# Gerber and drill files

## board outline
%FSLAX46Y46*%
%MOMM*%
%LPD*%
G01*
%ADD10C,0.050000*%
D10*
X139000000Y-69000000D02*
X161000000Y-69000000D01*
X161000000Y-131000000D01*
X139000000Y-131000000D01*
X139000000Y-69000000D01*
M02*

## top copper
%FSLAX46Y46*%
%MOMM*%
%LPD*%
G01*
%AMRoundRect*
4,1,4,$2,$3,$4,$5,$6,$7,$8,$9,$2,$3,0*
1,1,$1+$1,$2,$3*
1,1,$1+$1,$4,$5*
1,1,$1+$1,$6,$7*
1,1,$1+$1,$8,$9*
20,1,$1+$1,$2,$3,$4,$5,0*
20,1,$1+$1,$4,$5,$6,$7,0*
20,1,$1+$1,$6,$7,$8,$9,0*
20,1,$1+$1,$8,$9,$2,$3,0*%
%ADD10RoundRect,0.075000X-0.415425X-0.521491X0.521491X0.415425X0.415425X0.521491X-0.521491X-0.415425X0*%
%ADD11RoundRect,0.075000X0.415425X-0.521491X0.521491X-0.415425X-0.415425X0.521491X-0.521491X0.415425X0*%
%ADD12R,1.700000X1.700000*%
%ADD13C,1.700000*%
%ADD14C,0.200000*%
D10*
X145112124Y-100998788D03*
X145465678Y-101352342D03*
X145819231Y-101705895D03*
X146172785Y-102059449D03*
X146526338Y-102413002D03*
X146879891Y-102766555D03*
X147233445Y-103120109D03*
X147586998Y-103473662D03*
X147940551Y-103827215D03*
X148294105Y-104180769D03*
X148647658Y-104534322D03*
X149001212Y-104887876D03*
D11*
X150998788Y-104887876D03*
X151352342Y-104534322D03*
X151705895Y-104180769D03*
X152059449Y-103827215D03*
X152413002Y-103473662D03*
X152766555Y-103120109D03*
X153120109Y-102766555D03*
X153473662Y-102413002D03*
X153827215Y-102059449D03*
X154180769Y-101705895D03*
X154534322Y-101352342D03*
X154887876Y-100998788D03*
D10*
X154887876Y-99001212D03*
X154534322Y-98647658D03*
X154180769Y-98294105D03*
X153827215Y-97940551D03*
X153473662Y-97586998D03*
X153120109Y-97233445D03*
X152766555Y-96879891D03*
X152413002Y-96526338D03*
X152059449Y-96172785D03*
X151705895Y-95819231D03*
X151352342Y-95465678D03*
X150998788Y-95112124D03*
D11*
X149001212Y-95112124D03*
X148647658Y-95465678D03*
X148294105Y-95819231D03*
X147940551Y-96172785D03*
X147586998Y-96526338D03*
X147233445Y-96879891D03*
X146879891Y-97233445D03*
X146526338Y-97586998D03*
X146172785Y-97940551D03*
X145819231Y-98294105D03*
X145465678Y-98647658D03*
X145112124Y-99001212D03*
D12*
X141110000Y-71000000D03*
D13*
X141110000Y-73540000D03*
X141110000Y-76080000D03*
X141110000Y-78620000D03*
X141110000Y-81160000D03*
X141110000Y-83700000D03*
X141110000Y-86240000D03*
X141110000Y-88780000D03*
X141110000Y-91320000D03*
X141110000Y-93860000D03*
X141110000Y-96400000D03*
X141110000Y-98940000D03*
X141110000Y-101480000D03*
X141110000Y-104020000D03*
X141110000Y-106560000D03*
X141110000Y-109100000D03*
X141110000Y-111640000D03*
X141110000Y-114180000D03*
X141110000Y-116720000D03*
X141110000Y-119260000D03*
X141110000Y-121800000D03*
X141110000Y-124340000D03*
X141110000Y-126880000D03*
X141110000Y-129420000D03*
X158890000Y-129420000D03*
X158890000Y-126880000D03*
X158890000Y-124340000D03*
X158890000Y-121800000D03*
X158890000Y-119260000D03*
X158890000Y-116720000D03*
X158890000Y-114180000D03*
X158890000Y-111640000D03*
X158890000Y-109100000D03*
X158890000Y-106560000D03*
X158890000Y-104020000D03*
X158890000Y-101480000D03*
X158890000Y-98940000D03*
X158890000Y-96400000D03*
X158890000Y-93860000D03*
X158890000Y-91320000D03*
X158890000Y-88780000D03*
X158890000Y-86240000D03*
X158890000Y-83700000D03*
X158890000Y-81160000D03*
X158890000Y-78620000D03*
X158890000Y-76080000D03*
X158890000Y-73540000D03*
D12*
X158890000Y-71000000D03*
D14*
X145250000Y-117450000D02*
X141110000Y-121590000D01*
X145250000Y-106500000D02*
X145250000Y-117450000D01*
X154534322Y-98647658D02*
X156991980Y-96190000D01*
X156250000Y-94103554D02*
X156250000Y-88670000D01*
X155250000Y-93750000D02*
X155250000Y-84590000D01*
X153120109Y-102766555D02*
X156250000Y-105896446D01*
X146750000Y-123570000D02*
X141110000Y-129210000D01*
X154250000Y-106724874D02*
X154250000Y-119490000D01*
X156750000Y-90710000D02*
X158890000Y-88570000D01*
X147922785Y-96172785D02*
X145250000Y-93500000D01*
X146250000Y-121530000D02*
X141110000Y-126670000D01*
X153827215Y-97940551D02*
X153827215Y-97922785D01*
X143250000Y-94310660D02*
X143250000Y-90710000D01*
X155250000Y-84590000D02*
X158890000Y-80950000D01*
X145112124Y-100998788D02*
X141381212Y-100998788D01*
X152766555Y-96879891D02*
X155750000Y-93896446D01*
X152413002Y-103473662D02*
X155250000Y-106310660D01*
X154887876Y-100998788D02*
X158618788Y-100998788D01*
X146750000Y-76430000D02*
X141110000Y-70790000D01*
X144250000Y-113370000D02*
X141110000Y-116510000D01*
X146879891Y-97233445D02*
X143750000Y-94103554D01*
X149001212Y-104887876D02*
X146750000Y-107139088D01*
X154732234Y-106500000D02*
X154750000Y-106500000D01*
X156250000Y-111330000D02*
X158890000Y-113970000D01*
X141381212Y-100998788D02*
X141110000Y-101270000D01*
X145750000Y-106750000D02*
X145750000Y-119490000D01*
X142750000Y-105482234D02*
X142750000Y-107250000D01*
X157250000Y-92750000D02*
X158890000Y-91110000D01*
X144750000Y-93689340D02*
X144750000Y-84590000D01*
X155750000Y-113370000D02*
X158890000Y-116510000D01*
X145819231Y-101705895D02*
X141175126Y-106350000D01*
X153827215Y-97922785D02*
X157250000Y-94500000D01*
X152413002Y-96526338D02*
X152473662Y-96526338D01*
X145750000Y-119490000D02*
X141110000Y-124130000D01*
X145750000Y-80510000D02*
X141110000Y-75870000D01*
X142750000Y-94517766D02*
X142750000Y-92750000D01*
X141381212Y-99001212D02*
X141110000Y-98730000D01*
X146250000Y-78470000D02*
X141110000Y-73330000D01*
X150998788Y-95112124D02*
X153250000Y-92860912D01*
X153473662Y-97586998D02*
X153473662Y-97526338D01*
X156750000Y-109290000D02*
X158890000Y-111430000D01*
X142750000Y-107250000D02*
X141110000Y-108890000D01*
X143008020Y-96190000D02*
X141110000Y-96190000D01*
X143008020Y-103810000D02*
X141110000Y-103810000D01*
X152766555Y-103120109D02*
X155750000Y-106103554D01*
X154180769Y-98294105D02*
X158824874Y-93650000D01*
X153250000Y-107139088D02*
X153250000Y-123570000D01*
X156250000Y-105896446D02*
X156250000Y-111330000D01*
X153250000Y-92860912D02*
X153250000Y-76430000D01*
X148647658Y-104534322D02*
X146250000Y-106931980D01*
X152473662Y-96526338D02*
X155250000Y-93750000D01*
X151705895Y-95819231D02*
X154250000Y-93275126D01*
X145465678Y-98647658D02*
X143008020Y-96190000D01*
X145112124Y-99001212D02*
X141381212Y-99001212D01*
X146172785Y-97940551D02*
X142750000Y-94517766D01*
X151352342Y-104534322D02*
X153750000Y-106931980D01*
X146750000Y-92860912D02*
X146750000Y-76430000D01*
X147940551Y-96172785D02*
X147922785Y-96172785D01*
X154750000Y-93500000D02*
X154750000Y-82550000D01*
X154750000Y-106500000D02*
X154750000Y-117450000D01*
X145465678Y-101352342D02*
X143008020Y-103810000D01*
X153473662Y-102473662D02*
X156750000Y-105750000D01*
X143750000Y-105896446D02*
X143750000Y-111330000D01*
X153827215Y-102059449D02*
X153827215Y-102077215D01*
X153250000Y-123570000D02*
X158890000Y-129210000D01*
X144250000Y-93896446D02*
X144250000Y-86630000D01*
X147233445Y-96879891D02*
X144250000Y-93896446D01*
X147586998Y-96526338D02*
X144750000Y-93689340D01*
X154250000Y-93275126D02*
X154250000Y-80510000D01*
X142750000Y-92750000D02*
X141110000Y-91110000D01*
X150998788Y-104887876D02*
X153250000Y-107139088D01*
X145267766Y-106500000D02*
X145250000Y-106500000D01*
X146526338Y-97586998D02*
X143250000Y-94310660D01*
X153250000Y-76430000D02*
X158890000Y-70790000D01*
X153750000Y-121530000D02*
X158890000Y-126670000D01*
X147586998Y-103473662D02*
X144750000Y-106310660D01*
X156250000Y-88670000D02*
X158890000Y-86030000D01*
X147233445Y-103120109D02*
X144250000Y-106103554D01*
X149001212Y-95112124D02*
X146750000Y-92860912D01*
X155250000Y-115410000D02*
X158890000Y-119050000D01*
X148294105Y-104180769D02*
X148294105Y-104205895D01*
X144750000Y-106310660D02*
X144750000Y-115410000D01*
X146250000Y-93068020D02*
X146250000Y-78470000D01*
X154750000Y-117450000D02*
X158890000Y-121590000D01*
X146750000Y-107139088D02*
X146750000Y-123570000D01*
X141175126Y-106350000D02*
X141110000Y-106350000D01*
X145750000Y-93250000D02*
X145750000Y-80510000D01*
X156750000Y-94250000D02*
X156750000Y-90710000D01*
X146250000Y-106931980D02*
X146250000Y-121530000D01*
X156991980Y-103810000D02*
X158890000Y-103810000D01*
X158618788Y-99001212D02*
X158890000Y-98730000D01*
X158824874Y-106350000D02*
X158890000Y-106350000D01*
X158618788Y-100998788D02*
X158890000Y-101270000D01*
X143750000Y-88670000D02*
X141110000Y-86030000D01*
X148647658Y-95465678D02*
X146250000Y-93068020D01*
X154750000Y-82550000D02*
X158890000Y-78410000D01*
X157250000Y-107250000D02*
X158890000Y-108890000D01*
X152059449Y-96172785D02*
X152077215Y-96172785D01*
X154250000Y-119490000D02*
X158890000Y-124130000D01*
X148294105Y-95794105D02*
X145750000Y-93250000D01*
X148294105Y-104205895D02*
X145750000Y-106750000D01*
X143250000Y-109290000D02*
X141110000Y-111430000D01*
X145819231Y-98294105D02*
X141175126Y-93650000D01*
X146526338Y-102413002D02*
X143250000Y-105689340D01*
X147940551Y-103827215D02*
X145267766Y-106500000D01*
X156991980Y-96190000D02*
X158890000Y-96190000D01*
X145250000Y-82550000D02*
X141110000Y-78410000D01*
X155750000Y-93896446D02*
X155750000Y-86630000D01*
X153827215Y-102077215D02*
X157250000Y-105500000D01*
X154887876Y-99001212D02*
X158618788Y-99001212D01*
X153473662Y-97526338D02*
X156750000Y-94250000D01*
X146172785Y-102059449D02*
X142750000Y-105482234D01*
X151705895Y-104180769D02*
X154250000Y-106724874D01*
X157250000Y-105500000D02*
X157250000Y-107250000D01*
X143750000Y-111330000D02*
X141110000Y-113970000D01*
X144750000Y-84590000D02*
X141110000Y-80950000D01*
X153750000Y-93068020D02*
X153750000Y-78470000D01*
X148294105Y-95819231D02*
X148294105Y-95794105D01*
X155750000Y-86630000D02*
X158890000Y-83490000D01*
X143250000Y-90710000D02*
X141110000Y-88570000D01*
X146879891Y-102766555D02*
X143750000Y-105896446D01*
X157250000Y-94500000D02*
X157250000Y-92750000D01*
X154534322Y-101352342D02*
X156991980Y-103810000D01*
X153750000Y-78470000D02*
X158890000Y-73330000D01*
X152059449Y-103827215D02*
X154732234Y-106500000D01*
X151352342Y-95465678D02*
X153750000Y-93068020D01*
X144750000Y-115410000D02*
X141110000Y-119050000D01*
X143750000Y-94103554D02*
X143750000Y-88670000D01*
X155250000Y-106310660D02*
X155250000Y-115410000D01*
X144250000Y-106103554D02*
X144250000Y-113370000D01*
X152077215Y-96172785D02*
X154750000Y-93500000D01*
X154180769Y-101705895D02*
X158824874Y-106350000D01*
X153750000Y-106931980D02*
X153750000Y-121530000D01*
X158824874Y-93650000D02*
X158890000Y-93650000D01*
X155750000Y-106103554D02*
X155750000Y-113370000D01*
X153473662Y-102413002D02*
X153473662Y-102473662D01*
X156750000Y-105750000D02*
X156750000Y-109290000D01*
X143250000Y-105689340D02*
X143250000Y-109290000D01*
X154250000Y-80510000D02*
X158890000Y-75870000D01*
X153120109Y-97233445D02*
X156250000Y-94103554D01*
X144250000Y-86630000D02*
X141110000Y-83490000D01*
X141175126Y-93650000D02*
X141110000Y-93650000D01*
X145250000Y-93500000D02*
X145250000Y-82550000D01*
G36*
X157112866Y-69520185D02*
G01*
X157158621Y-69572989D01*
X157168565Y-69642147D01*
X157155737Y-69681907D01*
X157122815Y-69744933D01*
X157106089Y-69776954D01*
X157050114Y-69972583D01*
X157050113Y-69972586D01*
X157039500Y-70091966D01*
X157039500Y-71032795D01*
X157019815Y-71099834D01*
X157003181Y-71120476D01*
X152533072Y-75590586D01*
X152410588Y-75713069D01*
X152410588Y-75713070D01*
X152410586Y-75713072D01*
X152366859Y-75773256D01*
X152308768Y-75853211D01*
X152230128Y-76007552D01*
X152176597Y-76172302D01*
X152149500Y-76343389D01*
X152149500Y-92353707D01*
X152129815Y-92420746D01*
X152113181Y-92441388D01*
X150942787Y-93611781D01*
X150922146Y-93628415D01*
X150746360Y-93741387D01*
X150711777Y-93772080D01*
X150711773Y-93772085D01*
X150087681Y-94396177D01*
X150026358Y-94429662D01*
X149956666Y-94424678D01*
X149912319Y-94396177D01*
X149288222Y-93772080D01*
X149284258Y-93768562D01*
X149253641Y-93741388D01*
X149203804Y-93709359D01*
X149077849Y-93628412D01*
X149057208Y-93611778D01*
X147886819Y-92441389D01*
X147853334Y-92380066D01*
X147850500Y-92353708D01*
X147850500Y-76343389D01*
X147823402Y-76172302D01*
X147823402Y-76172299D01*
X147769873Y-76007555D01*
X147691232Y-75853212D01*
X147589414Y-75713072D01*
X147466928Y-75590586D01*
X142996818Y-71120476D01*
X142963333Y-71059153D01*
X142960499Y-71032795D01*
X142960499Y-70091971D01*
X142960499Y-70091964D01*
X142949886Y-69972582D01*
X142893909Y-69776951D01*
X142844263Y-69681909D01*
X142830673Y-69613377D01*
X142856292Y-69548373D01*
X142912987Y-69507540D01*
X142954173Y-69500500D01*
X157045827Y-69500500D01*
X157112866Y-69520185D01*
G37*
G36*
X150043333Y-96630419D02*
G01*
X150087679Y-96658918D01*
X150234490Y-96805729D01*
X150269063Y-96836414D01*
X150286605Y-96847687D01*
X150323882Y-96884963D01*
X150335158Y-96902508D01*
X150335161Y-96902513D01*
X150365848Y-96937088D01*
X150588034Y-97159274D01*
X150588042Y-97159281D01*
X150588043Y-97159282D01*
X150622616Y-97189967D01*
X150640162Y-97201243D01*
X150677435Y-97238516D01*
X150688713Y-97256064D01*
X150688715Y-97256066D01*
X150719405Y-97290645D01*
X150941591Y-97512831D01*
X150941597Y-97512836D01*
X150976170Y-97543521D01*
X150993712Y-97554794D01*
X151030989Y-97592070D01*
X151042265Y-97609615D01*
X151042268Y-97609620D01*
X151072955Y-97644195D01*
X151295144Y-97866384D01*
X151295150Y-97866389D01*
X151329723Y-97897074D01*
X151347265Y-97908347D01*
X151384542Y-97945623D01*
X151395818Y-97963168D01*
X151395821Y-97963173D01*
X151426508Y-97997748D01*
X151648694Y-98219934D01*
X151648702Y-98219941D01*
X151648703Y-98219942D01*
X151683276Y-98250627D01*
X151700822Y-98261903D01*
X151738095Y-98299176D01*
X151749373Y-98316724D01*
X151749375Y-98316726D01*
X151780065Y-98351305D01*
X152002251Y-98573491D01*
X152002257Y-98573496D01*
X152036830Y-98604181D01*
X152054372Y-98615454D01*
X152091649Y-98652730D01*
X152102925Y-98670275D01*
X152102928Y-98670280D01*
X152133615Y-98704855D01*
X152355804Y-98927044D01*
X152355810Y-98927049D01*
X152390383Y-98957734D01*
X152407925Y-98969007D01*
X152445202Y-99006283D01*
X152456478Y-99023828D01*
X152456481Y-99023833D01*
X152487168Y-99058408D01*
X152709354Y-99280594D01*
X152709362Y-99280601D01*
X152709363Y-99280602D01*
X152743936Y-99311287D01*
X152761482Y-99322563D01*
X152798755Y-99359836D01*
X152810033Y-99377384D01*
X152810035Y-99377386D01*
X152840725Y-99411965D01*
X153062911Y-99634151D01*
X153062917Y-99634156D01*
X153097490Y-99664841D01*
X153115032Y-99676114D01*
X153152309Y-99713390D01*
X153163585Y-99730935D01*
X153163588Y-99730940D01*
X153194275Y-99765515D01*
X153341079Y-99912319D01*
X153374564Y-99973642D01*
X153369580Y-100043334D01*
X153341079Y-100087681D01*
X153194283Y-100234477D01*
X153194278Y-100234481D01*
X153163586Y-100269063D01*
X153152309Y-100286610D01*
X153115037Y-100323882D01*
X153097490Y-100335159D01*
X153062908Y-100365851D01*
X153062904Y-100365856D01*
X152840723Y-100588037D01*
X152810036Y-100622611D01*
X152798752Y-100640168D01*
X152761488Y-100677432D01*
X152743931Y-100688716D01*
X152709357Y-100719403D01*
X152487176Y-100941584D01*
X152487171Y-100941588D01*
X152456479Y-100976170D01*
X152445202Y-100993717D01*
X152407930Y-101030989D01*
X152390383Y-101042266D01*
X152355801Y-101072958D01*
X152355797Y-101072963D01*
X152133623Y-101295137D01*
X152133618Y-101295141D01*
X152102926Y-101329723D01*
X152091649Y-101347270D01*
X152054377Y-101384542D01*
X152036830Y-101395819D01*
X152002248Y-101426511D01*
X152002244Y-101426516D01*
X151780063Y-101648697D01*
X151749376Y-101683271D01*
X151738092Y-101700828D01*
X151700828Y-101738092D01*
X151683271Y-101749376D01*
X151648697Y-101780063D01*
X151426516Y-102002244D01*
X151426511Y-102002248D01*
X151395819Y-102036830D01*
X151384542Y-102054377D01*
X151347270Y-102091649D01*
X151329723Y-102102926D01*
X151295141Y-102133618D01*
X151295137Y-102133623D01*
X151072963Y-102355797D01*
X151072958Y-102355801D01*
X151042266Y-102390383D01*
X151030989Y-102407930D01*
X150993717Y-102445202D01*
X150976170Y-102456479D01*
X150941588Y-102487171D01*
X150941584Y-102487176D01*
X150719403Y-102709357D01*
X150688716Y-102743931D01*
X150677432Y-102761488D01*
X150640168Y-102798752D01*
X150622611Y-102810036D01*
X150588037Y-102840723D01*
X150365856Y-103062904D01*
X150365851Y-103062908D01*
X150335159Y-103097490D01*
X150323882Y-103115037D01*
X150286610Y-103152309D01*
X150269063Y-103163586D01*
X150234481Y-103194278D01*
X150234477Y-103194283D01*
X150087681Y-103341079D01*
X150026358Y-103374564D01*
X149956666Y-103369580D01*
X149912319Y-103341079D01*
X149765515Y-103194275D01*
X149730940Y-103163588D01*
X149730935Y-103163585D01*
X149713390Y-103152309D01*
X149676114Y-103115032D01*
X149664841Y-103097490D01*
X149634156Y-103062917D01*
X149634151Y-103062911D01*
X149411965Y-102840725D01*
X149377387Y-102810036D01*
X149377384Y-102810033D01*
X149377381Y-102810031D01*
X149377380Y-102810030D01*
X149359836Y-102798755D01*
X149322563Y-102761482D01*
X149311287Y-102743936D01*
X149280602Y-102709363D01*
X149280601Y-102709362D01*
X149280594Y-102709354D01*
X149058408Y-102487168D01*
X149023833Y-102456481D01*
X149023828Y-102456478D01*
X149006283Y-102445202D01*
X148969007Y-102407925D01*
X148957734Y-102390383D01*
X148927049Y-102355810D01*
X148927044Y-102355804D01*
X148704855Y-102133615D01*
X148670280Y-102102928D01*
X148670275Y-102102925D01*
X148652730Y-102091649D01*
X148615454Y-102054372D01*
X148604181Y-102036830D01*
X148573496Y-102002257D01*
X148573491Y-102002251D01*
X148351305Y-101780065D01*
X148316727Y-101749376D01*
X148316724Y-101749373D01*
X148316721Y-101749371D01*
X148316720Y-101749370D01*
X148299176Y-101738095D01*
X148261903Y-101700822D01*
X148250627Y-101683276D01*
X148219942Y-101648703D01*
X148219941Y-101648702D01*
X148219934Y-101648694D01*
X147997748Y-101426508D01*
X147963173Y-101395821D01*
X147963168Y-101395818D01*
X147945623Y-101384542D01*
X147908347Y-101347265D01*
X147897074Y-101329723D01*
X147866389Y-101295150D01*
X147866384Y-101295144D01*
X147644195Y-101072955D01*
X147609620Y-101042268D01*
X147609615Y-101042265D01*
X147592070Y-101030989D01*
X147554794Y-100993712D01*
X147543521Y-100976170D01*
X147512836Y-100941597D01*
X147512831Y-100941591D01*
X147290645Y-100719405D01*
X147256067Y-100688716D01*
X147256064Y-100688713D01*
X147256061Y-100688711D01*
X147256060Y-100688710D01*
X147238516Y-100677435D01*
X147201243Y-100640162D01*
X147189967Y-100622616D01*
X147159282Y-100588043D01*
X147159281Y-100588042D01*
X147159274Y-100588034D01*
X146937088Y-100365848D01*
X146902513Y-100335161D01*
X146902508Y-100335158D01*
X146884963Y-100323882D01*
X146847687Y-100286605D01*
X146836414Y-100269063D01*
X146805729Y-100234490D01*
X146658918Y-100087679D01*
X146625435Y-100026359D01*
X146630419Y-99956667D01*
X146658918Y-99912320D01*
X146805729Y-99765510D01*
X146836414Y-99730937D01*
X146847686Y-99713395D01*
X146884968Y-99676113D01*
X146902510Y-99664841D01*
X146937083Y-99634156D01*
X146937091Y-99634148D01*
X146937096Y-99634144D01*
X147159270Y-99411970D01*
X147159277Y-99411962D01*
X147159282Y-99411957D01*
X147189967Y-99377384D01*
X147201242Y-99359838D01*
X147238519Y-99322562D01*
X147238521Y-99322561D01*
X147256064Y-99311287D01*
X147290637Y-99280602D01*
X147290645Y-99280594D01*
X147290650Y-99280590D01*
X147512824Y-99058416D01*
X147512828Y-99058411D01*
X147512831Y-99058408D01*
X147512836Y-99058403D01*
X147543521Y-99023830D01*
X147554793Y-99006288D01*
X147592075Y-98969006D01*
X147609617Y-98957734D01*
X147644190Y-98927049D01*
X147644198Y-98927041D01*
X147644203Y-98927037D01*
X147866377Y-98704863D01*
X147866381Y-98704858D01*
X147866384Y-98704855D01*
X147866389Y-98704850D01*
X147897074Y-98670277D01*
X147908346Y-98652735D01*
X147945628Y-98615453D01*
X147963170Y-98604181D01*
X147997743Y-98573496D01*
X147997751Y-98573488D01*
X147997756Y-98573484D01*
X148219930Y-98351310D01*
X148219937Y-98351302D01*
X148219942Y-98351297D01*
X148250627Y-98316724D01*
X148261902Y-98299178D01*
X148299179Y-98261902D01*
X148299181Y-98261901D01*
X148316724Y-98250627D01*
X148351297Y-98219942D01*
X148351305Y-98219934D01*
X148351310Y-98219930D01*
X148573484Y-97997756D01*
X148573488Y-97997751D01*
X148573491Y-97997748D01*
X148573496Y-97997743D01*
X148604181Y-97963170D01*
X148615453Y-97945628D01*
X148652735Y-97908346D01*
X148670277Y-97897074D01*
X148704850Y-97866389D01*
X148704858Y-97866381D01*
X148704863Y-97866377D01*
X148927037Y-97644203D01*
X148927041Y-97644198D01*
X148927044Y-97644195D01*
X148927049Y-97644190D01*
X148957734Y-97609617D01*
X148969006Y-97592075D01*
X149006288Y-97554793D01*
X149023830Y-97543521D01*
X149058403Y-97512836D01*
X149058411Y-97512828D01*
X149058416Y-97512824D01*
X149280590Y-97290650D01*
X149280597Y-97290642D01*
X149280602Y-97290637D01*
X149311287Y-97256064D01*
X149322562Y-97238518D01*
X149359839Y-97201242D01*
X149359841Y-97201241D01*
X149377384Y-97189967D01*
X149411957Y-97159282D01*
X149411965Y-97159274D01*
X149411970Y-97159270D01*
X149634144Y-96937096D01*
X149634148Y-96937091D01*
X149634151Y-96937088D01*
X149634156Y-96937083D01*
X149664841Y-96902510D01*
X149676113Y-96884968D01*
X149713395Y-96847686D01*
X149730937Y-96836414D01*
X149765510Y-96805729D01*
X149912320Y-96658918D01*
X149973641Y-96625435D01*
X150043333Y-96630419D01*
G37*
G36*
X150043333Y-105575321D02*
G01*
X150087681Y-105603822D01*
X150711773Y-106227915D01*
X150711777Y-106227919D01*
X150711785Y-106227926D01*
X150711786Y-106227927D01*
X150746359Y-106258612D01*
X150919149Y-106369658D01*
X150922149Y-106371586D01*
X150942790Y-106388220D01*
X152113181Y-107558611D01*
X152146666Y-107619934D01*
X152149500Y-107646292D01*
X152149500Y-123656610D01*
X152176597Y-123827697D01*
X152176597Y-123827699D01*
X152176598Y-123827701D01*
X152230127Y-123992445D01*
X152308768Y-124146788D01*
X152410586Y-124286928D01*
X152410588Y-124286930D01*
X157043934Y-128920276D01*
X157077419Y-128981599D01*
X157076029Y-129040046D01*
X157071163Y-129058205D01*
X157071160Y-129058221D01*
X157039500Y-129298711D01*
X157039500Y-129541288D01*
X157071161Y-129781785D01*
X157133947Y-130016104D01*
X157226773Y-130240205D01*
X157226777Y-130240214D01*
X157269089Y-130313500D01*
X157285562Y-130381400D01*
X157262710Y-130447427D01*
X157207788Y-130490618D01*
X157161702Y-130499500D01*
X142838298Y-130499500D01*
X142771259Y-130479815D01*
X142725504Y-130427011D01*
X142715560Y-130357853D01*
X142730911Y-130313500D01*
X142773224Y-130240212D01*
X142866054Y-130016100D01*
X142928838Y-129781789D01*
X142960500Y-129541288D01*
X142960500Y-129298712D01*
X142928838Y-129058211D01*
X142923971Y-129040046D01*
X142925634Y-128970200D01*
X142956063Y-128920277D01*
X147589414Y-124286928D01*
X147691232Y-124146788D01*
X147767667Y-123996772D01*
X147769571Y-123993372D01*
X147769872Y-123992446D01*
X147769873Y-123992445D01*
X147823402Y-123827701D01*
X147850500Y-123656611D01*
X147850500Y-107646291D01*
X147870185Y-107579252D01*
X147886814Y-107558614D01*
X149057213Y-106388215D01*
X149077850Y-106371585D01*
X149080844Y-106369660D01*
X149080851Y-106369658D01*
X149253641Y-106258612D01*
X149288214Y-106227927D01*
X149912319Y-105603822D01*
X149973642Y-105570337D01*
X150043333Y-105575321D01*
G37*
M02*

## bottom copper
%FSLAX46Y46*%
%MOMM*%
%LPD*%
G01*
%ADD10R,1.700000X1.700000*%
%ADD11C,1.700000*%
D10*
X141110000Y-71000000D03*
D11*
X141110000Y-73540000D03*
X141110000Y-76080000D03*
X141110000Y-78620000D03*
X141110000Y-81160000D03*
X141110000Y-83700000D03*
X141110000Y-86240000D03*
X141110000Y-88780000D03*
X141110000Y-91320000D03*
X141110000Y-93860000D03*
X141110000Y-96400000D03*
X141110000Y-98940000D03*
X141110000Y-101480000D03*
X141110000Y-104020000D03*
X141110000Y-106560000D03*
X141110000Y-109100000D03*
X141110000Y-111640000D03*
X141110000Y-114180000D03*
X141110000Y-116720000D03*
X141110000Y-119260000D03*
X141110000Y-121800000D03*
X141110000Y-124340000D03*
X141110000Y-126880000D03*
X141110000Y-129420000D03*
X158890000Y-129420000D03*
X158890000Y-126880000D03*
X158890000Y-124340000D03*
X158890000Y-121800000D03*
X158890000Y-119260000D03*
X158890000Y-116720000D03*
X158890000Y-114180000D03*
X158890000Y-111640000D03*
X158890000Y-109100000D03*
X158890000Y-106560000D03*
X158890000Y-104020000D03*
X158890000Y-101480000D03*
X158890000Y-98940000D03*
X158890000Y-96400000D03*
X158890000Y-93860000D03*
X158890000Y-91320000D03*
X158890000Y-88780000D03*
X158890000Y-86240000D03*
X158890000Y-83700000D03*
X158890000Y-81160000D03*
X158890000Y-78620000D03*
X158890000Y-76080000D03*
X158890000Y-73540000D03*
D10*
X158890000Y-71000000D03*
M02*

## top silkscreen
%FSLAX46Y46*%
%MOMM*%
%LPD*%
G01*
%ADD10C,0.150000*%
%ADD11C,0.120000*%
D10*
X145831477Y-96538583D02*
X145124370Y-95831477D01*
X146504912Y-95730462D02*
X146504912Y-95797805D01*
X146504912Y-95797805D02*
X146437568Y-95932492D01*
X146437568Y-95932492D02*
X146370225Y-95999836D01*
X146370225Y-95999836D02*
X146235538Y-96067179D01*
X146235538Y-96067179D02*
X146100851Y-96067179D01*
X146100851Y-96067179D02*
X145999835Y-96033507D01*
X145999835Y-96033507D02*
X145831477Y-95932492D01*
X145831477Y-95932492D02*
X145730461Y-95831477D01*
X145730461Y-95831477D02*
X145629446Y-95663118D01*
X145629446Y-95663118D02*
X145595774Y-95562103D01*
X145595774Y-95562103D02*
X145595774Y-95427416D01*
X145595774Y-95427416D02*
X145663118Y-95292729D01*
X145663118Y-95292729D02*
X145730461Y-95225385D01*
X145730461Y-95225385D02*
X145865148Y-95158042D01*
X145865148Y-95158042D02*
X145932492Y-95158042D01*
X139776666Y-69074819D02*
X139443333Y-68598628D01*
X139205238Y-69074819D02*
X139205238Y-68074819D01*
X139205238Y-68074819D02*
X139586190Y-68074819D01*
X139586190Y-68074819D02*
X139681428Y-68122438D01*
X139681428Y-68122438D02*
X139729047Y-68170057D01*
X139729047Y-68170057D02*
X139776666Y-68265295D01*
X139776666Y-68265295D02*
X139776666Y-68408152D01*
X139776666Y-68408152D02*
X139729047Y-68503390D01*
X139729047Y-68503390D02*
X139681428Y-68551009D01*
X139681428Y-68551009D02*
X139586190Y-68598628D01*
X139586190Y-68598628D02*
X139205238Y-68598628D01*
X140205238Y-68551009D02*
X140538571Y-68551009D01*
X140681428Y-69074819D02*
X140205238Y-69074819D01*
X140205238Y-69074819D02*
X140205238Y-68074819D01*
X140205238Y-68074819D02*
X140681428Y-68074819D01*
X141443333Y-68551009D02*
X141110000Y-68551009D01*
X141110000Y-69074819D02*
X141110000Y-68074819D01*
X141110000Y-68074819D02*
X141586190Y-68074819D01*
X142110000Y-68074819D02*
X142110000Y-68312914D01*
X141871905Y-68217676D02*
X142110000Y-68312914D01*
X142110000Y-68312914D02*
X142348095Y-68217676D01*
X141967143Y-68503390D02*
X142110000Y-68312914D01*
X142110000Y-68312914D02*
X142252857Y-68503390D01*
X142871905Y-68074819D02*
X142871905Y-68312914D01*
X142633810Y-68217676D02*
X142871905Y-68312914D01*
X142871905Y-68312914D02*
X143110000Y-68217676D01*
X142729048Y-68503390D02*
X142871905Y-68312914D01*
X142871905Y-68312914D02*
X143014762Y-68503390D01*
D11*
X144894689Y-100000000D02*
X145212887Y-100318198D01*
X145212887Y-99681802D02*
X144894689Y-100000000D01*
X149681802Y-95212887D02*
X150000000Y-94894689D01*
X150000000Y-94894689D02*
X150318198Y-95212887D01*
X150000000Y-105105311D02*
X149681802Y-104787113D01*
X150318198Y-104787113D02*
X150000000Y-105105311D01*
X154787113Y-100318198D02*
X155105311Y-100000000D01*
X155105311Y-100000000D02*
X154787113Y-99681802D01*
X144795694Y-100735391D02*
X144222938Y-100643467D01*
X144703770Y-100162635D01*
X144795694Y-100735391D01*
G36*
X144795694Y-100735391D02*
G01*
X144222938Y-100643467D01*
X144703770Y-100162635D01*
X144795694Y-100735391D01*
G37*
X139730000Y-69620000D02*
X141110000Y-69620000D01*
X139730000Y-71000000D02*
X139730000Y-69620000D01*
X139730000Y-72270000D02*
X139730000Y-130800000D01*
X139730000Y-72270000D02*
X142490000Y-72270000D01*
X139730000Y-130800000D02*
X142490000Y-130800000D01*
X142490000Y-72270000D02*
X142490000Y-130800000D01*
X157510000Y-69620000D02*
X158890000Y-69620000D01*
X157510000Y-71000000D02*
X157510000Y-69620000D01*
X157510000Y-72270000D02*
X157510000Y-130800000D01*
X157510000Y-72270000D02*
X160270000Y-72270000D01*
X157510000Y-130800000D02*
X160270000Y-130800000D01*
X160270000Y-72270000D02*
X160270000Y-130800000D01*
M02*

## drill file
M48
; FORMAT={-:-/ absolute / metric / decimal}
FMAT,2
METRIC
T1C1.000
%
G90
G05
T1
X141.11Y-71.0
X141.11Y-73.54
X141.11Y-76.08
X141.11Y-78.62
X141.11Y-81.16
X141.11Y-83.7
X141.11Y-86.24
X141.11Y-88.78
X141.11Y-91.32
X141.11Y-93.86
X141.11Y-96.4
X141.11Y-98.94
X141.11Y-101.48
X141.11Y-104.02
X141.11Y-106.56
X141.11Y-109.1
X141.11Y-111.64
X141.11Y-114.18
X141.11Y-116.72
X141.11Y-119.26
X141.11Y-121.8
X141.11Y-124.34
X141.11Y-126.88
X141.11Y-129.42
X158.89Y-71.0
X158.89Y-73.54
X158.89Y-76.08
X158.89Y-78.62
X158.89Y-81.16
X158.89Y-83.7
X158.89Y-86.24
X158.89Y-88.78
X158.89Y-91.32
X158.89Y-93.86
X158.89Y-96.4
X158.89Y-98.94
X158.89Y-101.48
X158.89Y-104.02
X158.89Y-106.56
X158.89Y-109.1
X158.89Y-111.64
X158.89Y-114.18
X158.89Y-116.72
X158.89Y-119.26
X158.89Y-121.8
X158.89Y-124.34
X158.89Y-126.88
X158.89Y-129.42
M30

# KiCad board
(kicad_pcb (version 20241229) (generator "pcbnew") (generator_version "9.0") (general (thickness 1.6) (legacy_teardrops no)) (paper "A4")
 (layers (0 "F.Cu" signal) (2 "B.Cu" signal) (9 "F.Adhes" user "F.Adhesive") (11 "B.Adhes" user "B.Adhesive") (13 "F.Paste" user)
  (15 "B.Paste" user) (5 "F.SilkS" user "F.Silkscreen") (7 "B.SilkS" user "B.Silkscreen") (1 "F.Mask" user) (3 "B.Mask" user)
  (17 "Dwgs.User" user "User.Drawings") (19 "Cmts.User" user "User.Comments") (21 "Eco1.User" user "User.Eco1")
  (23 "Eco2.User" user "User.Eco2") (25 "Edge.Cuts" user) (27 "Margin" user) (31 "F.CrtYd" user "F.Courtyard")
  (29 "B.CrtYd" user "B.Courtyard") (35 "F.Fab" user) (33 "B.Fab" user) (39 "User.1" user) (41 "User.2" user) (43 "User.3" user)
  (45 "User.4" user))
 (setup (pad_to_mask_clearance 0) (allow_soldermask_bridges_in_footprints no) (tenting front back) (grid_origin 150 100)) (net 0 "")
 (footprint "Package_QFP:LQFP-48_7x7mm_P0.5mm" (layer "F.Cu") (at 150 100 45)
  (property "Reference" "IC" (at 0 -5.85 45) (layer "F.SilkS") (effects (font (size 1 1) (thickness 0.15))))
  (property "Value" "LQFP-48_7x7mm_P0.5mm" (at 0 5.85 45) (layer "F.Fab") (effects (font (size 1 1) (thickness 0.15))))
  (fp_line (start -3.61 -3.61) (end -3.61 -3.16) (stroke (width 0.12) (type solid)) (layer "F.SilkS"))
  (fp_line (start -3.16 -3.61) (end -3.61 -3.61) (stroke (width 0.12) (type solid)) (layer "F.SilkS"))
  (fp_line (start 3.16 -3.61) (end 3.61 -3.61) (stroke (width 0.12) (type solid)) (layer "F.SilkS"))
  (fp_line (start 3.61 -3.61) (end 3.61 -3.16) (stroke (width 0.12) (type solid)) (layer "F.SilkS"))
  (fp_line (start -3.61 3.61) (end -3.61 3.16) (stroke (width 0.12) (type solid)) (layer "F.SilkS"))
  (fp_line (start -3.16 3.61) (end -3.61 3.61) (stroke (width 0.12) (type solid)) (layer "F.SilkS"))
  (fp_line (start 3.16 3.61) (end 3.61 3.61) (stroke (width 0.12) (type solid)) (layer "F.SilkS"))
  (fp_line (start 3.61 3.61) (end 3.61 3.16) (stroke (width 0.12) (type solid)) (layer "F.SilkS"))
  (fp_poly (pts (xy -4.2 -3.16) (xy -4.54 -3.63) (xy -3.86 -3.63)) (stroke (width 0.12) (type solid)) (fill yes) (layer "F.SilkS"))
  (pad "1" smd roundrect (at -4.1625 -2.75 45) (size 1.475 0.3) (layers "F.Cu" "F.Mask" "F.Paste") (roundrect_rratio 0.25))
  (pad "2" smd roundrect (at -4.1625 -2.25 45) (size 1.475 0.3) (layers "F.Cu" "F.Mask" "F.Paste") (roundrect_rratio 0.25))
  (pad "3" smd roundrect (at -4.1625 -1.75 45) (size 1.475 0.3) (layers "F.Cu" "F.Mask" "F.Paste") (roundrect_rratio 0.25))
  (pad "4" smd roundrect (at -4.1625 -1.249999 45) (size 1.475 0.3) (layers "F.Cu" "F.Mask" "F.Paste") (roundrect_rratio 0.25))
  (pad "5" smd roundrect (at -4.1625 -0.75 45) (size 1.475 0.3) (layers "F.Cu" "F.Mask" "F.Paste") (roundrect_rratio 0.25))
  (pad "6" smd roundrect (at -4.1625 -0.25 45) (size 1.475 0.3) (layers "F.Cu" "F.Mask" "F.Paste") (roundrect_rratio 0.25))
  (pad "7" smd roundrect (at -4.1625 0.25 45) (size 1.475 0.3) (layers "F.Cu" "F.Mask" "F.Paste") (roundrect_rratio 0.25))
  (pad "8" smd roundrect (at -4.1625 0.75 45) (size 1.475 0.3) (layers "F.Cu" "F.Mask" "F.Paste") (roundrect_rratio 0.25))
  (pad "9" smd roundrect (at -4.1625 1.249999 45) (size 1.475 0.3) (layers "F.Cu" "F.Mask" "F.Paste") (roundrect_rratio 0.25))
  (pad "10" smd roundrect (at -4.1625 1.75 45) (size 1.475 0.3) (layers "F.Cu" "F.Mask" "F.Paste") (roundrect_rratio 0.25))
  (pad "11" smd roundrect (at -4.1625 2.25 45) (size 1.475 0.3) (layers "F.Cu" "F.Mask" "F.Paste") (roundrect_rratio 0.25))
  (pad "12" smd roundrect (at -4.1625 2.75 45) (size 1.475 0.3) (layers "F.Cu" "F.Mask" "F.Paste") (roundrect_rratio 0.25))
  (pad "13" smd roundrect (at -2.75 4.1625 45) (size 0.3 1.475) (layers "F.Cu" "F.Mask" "F.Paste") (roundrect_rratio 0.25))
  (pad "14" smd roundrect (at -2.25 4.1625 45) (size 0.3 1.475) (layers "F.Cu" "F.Mask" "F.Paste") (roundrect_rratio 0.25))
  (pad "15" smd roundrect (at -1.75 4.1625 45) (size 0.3 1.475) (layers "F.Cu" "F.Mask" "F.Paste") (roundrect_rratio 0.25))
  (pad "16" smd roundrect (at -1.249999 4.1625 45) (size 0.3 1.475) (layers "F.Cu" "F.Mask" "F.Paste") (roundrect_rratio 0.25))
  (pad "17" smd roundrect (at -0.75 4.1625 45) (size 0.3 1.475) (layers "F.Cu" "F.Mask" "F.Paste") (roundrect_rratio 0.25))
  (pad "18" smd roundrect (at -0.25 4.1625 45) (size 0.3 1.475) (layers "F.Cu" "F.Mask" "F.Paste") (roundrect_rratio 0.25))
  (pad "19" smd roundrect (at 0.25 4.1625 45) (size 0.3 1.475) (layers "F.Cu" "F.Mask" "F.Paste") (roundrect_rratio 0.25))
  (pad "20" smd roundrect (at 0.75 4.1625 45) (size 0.3 1.475) (layers "F.Cu" "F.Mask" "F.Paste") (roundrect_rratio 0.25))
  (pad "21" smd roundrect (at 1.249999 4.1625 45) (size 0.3 1.475) (layers "F.Cu" "F.Mask" "F.Paste") (roundrect_rratio 0.25))
  (pad "22" smd roundrect (at 1.75 4.1625 45) (size 0.3 1.475) (layers "F.Cu" "F.Mask" "F.Paste") (roundrect_rratio 0.25))
  (pad "23" smd roundrect (at 2.25 4.1625 45) (size 0.3 1.475) (layers "F.Cu" "F.Mask" "F.Paste") (roundrect_rratio 0.25))
  (pad "24" smd roundrect (at 2.75 4.1625 45) (size 0.3 1.475) (layers "F.Cu" "F.Mask" "F.Paste") (roundrect_rratio 0.25))
  (pad "25" smd roundrect (at 4.1625 2.75 45) (size 1.475 0.3) (layers "F.Cu" "F.Mask" "F.Paste") (roundrect_rratio 0.25))
  (pad "26" smd roundrect (at 4.1625 2.25 45) (size 1.475 0.3) (layers "F.Cu" "F.Mask" "F.Paste") (roundrect_rratio 0.25))
  (pad "27" smd roundrect (at 4.1625 1.75 45) (size 1.475 0.3) (layers "F.Cu" "F.Mask" "F.Paste") (roundrect_rratio 0.25))
  (pad "28" smd roundrect (at 4.1625 1.249999 45) (size 1.475 0.3) (layers "F.Cu" "F.Mask" "F.Paste") (roundrect_rratio 0.25))
  (pad "29" smd roundrect (at 4.1625 0.75 45) (size 1.475 0.3) (layers "F.Cu" "F.Mask" "F.Paste") (roundrect_rratio 0.25))
  (pad "30" smd roundrect (at 4.1625 0.25 45) (size 1.475 0.3) (layers "F.Cu" "F.Mask" "F.Paste") (roundrect_rratio 0.25))
  (pad "31" smd roundrect (at 4.1625 -0.25 45) (size 1.475 0.3) (layers "F.Cu" "F.Mask" "F.Paste") (roundrect_rratio 0.25))
  (pad "32" smd roundrect (at 4.1625 -0.75 45) (size 1.475 0.3) (layers "F.Cu" "F.Mask" "F.Paste") (roundrect_rratio 0.25))
  (pad "33" smd roundrect (at 4.1625 -1.249999 45) (size 1.475 0.3) (layers "F.Cu" "F.Mask" "F.Paste") (roundrect_rratio 0.25))
  (pad "34" smd roundrect (at 4.1625 -1.75 45) (size 1.475 0.3) (layers "F.Cu" "F.Mask" "F.Paste") (roundrect_rratio 0.25))
  (pad "35" smd roundrect (at 4.1625 -2.25 45) (size 1.475 0.3) (layers "F.Cu" "F.Mask" "F.Paste") (roundrect_rratio 0.25))
  (pad "36" smd roundrect (at 4.1625 -2.75 45) (size 1.475 0.3) (layers "F.Cu" "F.Mask" "F.Paste") (roundrect_rratio 0.25))
  (pad "37" smd roundrect (at 2.75 -4.1625 45) (size 0.3 1.475) (layers "F.Cu" "F.Mask" "F.Paste") (roundrect_rratio 0.25))
  (pad "38" smd roundrect (at 2.25 -4.1625 45) (size 0.3 1.475) (layers "F.Cu" "F.Mask" "F.Paste") (roundrect_rratio 0.25))
  (pad "39" smd roundrect (at 1.75 -4.1625 45) (size 0.3 1.475) (layers "F.Cu" "F.Mask" "F.Paste") (roundrect_rratio 0.25))
  (pad "40" smd roundrect (at 1.249999 -4.1625 45) (size 0.3 1.475) (layers "F.Cu" "F.Mask" "F.Paste") (roundrect_rratio 0.25))
  (pad "41" smd roundrect (at 0.75 -4.1625 45) (size 0.3 1.475) (layers "F.Cu" "F.Mask" "F.Paste") (roundrect_rratio 0.25))
  (pad "42" smd roundrect (at 0.25 -4.1625 45) (size 0.3 1.475) (layers "F.Cu" "F.Mask" "F.Paste") (roundrect_rratio 0.25))
  (pad "43" smd roundrect (at -0.25 -4.1625 45) (size 0.3 1.475) (layers "F.Cu" "F.Mask" "F.Paste") (roundrect_rratio 0.25))
  (pad "44" smd roundrect (at -0.75 -4.1625 45) (size 0.3 1.475) (layers "F.Cu" "F.Mask" "F.Paste") (roundrect_rratio 0.25))
  (pad "45" smd roundrect (at -1.249999 -4.1625 45) (size 0.3 1.475) (layers "F.Cu" "F.Mask" "F.Paste") (roundrect_rratio 0.25))
  (pad "46" smd roundrect (at -1.75 -4.1625 45) (size 0.3 1.475) (layers "F.Cu" "F.Mask" "F.Paste") (roundrect_rratio 0.25))
  (pad "47" smd roundrect (at -2.25 -4.1625 45) (size 0.3 1.475) (layers "F.Cu" "F.Mask" "F.Paste") (roundrect_rratio 0.25))
  (pad "48" smd roundrect (at -2.75 -4.1625 45) (size 0.3 1.475) (layers "F.Cu" "F.Mask" "F.Paste") (roundrect_rratio 0.25)))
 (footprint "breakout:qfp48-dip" (layer "F.Cu") (at 150 71)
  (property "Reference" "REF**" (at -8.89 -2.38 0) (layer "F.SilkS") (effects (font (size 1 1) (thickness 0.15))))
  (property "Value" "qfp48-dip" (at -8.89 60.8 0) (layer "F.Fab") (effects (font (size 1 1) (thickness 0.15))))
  (fp_line (start -10.27 -1.38) (end -8.89 -1.38) (stroke (width 0.12) (type solid)) (layer "F.SilkS"))
  (fp_line (start -10.27 0) (end -10.27 -1.38) (stroke (width 0.12) (type solid)) (layer "F.SilkS"))
  (fp_line (start -10.27 1.27) (end -10.27 59.8) (stroke (width 0.12) (type solid)) (layer "F.SilkS"))
  (fp_line (start -10.27 1.27) (end -7.51 1.27) (stroke (width 0.12) (type solid)) (layer "F.SilkS"))
  (fp_line (start -10.27 59.8) (end -7.51 59.8) (stroke (width 0.12) (type solid)) (layer "F.SilkS"))
  (fp_line (start -7.51 1.27) (end -7.51 59.8) (stroke (width 0.12) (type solid)) (layer "F.SilkS"))
  (fp_line (start 7.51 -1.38) (end 8.89 -1.38) (stroke (width 0.12) (type solid)) (layer "F.SilkS"))
  (fp_line (start 7.51 0) (end 7.51 -1.38) (stroke (width 0.12) (type solid)) (layer "F.SilkS"))
  (fp_line (start 7.51 1.27) (end 7.51 59.8) (stroke (width 0.12) (type solid)) (layer "F.SilkS"))
  (fp_line (start 7.51 1.27) (end 10.27 1.27) (stroke (width 0.12) (type solid)) (layer "F.SilkS"))
  (fp_line (start 7.51 59.8) (end 10.27 59.8) (stroke (width 0.12) (type solid)) (layer "F.SilkS"))
  (fp_line (start 10.27 1.27) (end 10.27 59.8) (stroke (width 0.12) (type solid)) (layer "F.SilkS"))
  (pad "1" thru_hole rect (at -8.89 0) (size 1.7 1.7) (drill 1) (layers "*.Cu" "*.Mask") (remove_unused_layers no))
  (pad "2" thru_hole circle (at -8.89 2.54) (size 1.7 1.7) (drill 1) (layers "*.Cu" "*.Mask") (remove_unused_layers no))
  (pad "3" thru_hole circle (at -8.89 5.08) (size 1.7 1.7) (drill 1) (layers "*.Cu" "*.Mask") (remove_unused_layers no))
  (pad "4" thru_hole circle (at -8.89 7.62) (size 1.7 1.7) (drill 1) (layers "*.Cu" "*.Mask") (remove_unused_layers no))
  (pad "5" thru_hole circle (at -8.89 10.16) (size 1.7 1.7) (drill 1) (layers "*.Cu" "*.Mask") (remove_unused_layers no))
  (pad "6" thru_hole circle (at -8.89 12.7) (size 1.7 1.7) (drill 1) (layers "*.Cu" "*.Mask") (remove_unused_layers no))
  (pad "7" thru_hole circle (at -8.89 15.24) (size 1.7 1.7) (drill 1) (layers "*.Cu" "*.Mask") (remove_unused_layers no))
  (pad "8" thru_hole circle (at -8.89 17.78) (size 1.7 1.7) (drill 1) (layers "*.Cu" "*.Mask") (remove_unused_layers no))
  (pad "9" thru_hole circle (at -8.89 20.32) (size 1.7 1.7) (drill 1) (layers "*.Cu" "*.Mask") (remove_unused_layers no))
  (pad "10" thru_hole circle (at -8.89 22.86) (size 1.7 1.7) (drill 1) (layers "*.Cu" "*.Mask") (remove_unused_layers no))
  (pad "11" thru_hole circle (at -8.89 25.4) (size 1.7 1.7) (drill 1) (layers "*.Cu" "*.Mask") (remove_unused_layers no))
  (pad "12" thru_hole circle (at -8.89 27.94) (size 1.7 1.7) (drill 1) (layers "*.Cu" "*.Mask") (remove_unused_layers no))
  (pad "13" thru_hole circle (at -8.89 30.48) (size 1.7 1.7) (drill 1) (layers "*.Cu" "*.Mask") (remove_unused_layers no))
  (pad "14" thru_hole circle (at -8.89 33.02) (size 1.7 1.7) (drill 1) (layers "*.Cu" "*.Mask") (remove_unused_layers no))
  (pad "15" thru_hole circle (at -8.89 35.56) (size 1.7 1.7) (drill 1) (layers "*.Cu" "*.Mask") (remove_unused_layers no))
  (pad "16" thru_hole circle (at -8.89 38.1) (size 1.7 1.7) (drill 1) (layers "*.Cu" "*.Mask") (remove_unused_layers no))
  (pad "17" thru_hole circle (at -8.89 40.64) (size 1.7 1.7) (drill 1) (layers "*.Cu" "*.Mask") (remove_unused_layers no))
  (pad "18" thru_hole circle (at -8.89 43.18) (size 1.7 1.7) (drill 1) (layers "*.Cu" "*.Mask") (remove_unused_layers no))
  (pad "19" thru_hole circle (at -8.89 45.72) (size 1.7 1.7) (drill 1) (layers "*.Cu" "*.Mask") (remove_unused_layers no))
  (pad "20" thru_hole circle (at -8.89 48.26) (size 1.7 1.7) (drill 1) (layers "*.Cu" "*.Mask") (remove_unused_layers no))
  (pad "21" thru_hole circle (at -8.89 50.8) (size 1.7 1.7) (drill 1) (layers "*.Cu" "*.Mask") (remove_unused_layers no))
  (pad "22" thru_hole circle (at -8.89 53.34) (size 1.7 1.7) (drill 1) (layers "*.Cu" "*.Mask") (remove_unused_layers no))
  (pad "23" thru_hole circle (at -8.89 55.88) (size 1.7 1.7) (drill 1) (layers "*.Cu" "*.Mask") (remove_unused_layers no))
  (pad "24" thru_hole circle (at -8.89 58.42) (size 1.7 1.7) (drill 1) (layers "*.Cu" "*.Mask") (remove_unused_layers no))
  (pad "25" thru_hole circle (at 8.89 58.42) (size 1.7 1.7) (drill 1) (layers "*.Cu" "*.Mask") (remove_unused_layers no))
  (pad "26" thru_hole circle (at 8.89 55.88) (size 1.7 1.7) (drill 1) (layers "*.Cu" "*.Mask") (remove_unused_layers no))
  (pad "27" thru_hole circle (at 8.89 53.34) (size 1.7 1.7) (drill 1) (layers "*.Cu" "*.Mask") (remove_unused_layers no))
  (pad "28" thru_hole circle (at 8.89 50.8) (size 1.7 1.7) (drill 1) (layers "*.Cu" "*.Mask") (remove_unused_layers no))
  (pad "29" thru_hole circle (at 8.89 48.26) (size 1.7 1.7) (drill 1) (layers "*.Cu" "*.Mask") (remove_unused_layers no))
  (pad "30" thru_hole circle (at 8.89 45.72) (size 1.7 1.7) (drill 1) (layers "*.Cu" "*.Mask") (remove_unused_layers no))
  (pad "31" thru_hole circle (at 8.89 43.18) (size 1.7 1.7) (drill 1) (layers "*.Cu" "*.Mask") (remove_unused_layers no))
  (pad "32" thru_hole circle (at 8.89 40.64) (size 1.7 1.7) (drill 1) (layers "*.Cu" "*.Mask") (remove_unused_layers no))
  (pad "33" thru_hole circle (at 8.89 38.1) (size 1.7 1.7) (drill 1) (layers "*.Cu" "*.Mask") (remove_unused_layers no))
  (pad "34" thru_hole circle (at 8.89 35.56) (size 1.7 1.7) (drill 1) (layers "*.Cu" "*.Mask") (remove_unused_layers no))
  (pad "35" thru_hole circle (at 8.89 33.02) (size 1.7 1.7) (drill 1) (layers "*.Cu" "*.Mask") (remove_unused_layers no))
  (pad "36" thru_hole circle (at 8.89 30.48) (size 1.7 1.7) (drill 1) (layers "*.Cu" "*.Mask") (remove_unused_layers no))
  (pad "37" thru_hole circle (at 8.89 27.94) (size 1.7 1.7) (drill 1) (layers "*.Cu" "*.Mask") (remove_unused_layers no))
  (pad "38" thru_hole circle (at 8.89 25.4) (size 1.7 1.7) (drill 1) (layers "*.Cu" "*.Mask") (remove_unused_layers no))
  (pad "39" thru_hole circle (at 8.89 22.86) (size 1.7 1.7) (drill 1) (layers "*.Cu" "*.Mask") (remove_unused_layers no))
  (pad "40" thru_hole circle (at 8.89 20.32) (size 1.7 1.7) (drill 1) (layers "*.Cu" "*.Mask") (remove_unused_layers no))
  (pad "41" thru_hole circle (at 8.89 17.78) (size 1.7 1.7) (drill 1) (layers "*.Cu" "*.Mask") (remove_unused_layers no))
  (pad "42" thru_hole circle (at 8.89 15.24) (size 1.7 1.7) (drill 1) (layers "*.Cu" "*.Mask") (remove_unused_layers no))
  (pad "43" thru_hole circle (at 8.89 12.7) (size 1.7 1.7) (drill 1) (layers "*.Cu" "*.Mask") (remove_unused_layers no))
  (pad "44" thru_hole circle (at 8.89 10.16) (size 1.7 1.7) (drill 1) (layers "*.Cu" "*.Mask") (remove_unused_layers no))
  (pad "45" thru_hole circle (at 8.89 7.62) (size 1.7 1.7) (drill 1) (layers "*.Cu" "*.Mask") (remove_unused_layers no))
  (pad "46" thru_hole circle (at 8.89 5.08) (size 1.7 1.7) (drill 1) (layers "*.Cu" "*.Mask") (remove_unused_layers no))
  (pad "47" thru_hole circle (at 8.89 2.54) (size 1.7 1.7) (drill 1) (layers "*.Cu" "*.Mask") (remove_unused_layers no))
  (pad "48" thru_hole rect (at 8.89 0) (size 1.7 1.7) (drill 1) (layers "*.Cu" "*.Mask") (remove_unused_layers no)))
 (gr_rect (start 139 69) (end 161 131) (stroke (width 0.05) (type default)) (fill no) (layer "Edge.Cuts"))
 (segment (start 145.25 117.45) (end 141.11 121.59) (width 0.2) (layer "F.Cu") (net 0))
 (segment (start 145.25 106.5) (end 145.25 117.45) (width 0.2) (layer "F.Cu") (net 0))
 (segment (start 154.534322 98.647658) (end 156.99198 96.19) (width 0.2) (layer "F.Cu") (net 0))
 (segment (start 156.25 94.103554) (end 156.25 88.67) (width 0.2) (layer "F.Cu") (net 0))
 (segment (start 155.25 93.75) (end 155.25 84.59) (width 0.2) (layer "F.Cu") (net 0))
 (segment (start 153.120109 102.766555) (end 156.25 105.896446) (width 0.2) (layer "F.Cu") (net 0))
 (segment (start 146.75 123.57) (end 141.11 129.21) (width 0.2) (layer "F.Cu") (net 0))
 (segment (start 154.25 106.724874) (end 154.25 119.49) (width 0.2) (layer "F.Cu") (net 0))
 (segment (start 156.75 90.71) (end 158.89 88.57) (width 0.2) (layer "F.Cu") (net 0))
 (segment (start 147.922785 96.172785) (end 145.25 93.5) (width 0.2) (layer "F.Cu") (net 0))
 (segment (start 146.25 121.53) (end 141.11 126.67) (width 0.2) (layer "F.Cu") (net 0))
 (segment (start 153.827215 97.940551) (end 153.827215 97.922785) (width 0.2) (layer "F.Cu") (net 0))
 (segment (start 143.25 94.31066) (end 143.25 90.71) (width 0.2) (layer "F.Cu") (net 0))
 (segment (start 155.25 84.59) (end 158.89 80.95) (width 0.2) (layer "F.Cu") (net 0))
 (segment (start 145.112124 100.998788) (end 141.381212 100.998788) (width 0.2) (layer "F.Cu") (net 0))
 (segment (start 152.766555 96.879891) (end 155.75 93.896446) (width 0.2) (layer "F.Cu") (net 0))
 (segment (start 152.413002 103.473662) (end 155.25 106.31066) (width 0.2) (layer "F.Cu") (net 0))
 (segment (start 154.887876 100.998788) (end 158.618788 100.998788) (width 0.2) (layer "F.Cu") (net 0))
 (segment (start 146.75 76.43) (end 141.11 70.79) (width 0.2) (layer "F.Cu") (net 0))
 (segment (start 144.25 113.37) (end 141.11 116.51) (width 0.2) (layer "F.Cu") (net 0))
 (segment (start 146.879891 97.233445) (end 143.75 94.103554) (width 0.2) (layer "F.Cu") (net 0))
 (segment (start 149.001212 104.887876) (end 146.75 107.139088) (width 0.2) (layer "F.Cu") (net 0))
 (segment (start 154.732234 106.5) (end 154.75 106.5) (width 0.2) (layer "F.Cu") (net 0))
 (segment (start 156.25 111.33) (end 158.89 113.97) (width 0.2) (layer "F.Cu") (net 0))
 (segment (start 141.381212 100.998788) (end 141.11 101.27) (width 0.2) (layer "F.Cu") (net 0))
 (segment (start 145.75 106.75) (end 145.75 119.49) (width 0.2) (layer "F.Cu") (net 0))
 (segment (start 142.75 105.482234) (end 142.75 107.25) (width 0.2) (layer "F.Cu") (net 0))
 (segment (start 157.25 92.75) (end 158.89 91.11) (width 0.2) (layer "F.Cu") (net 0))
 (segment (start 144.75 93.68934) (end 144.75 84.59) (width 0.2) (layer "F.Cu") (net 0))
 (segment (start 155.75 113.37) (end 158.89 116.51) (width 0.2) (layer "F.Cu") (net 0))
 (segment (start 145.819231 101.705895) (end 141.175126 106.35) (width 0.2) (layer "F.Cu") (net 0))
 (segment (start 153.827215 97.922785) (end 157.25 94.5) (width 0.2) (layer "F.Cu") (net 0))
 (segment (start 152.413002 96.526338) (end 152.473662 96.526338) (width 0.2) (layer "F.Cu") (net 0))
 (segment (start 145.75 119.49) (end 141.11 124.13) (width 0.2) (layer "F.Cu") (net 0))
 (segment (start 145.75 80.51) (end 141.11 75.87) (width 0.2) (layer "F.Cu") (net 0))
 (segment (start 142.75 94.517766) (end 142.75 92.75) (width 0.2) (layer "F.Cu") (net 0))
 (segment (start 141.381212 99.001212) (end 141.11 98.73) (width 0.2) (layer "F.Cu") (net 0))
 (segment (start 146.25 78.47) (end 141.11 73.33) (width 0.2) (layer "F.Cu") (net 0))
 (segment (start 150.998788 95.112124) (end 153.25 92.860912) (width 0.2) (layer "F.Cu") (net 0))
 (segment (start 153.473662 97.586998) (end 153.473662 97.526338) (width 0.2) (layer "F.Cu") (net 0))
 (segment (start 156.75 109.29) (end 158.89 111.43) (width 0.2) (layer "F.Cu") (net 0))
 (segment (start 142.75 107.25) (end 141.11 108.89) (width 0.2) (layer "F.Cu") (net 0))
 (segment (start 143.00802 96.19) (end 141.11 96.19) (width 0.2) (layer "F.Cu") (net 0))
 (segment (start 143.00802 103.81) (end 141.11 103.81) (width 0.2) (layer "F.Cu") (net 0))
 (segment (start 152.766555 103.120109) (end 155.75 106.103554) (width 0.2) (layer "F.Cu") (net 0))
 (segment (start 154.180769 98.294105) (end 158.824874 93.65) (width 0.2) (layer "F.Cu") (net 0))
 (segment (start 153.25 107.139088) (end 153.25 123.57) (width 0.2) (layer "F.Cu") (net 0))
 (segment (start 156.25 105.896446) (end 156.25 111.33) (width 0.2) (layer "F.Cu") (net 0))
 (segment (start 153.25 92.860912) (end 153.25 76.43) (width 0.2) (layer "F.Cu") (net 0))
 (segment (start 148.647658 104.534322) (end 146.25 106.93198) (width 0.2) (layer "F.Cu") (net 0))
 (segment (start 152.473662 96.526338) (end 155.25 93.75) (width 0.2) (layer "F.Cu") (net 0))
 (segment (start 151.705895 95.819231) (end 154.25 93.275126) (width 0.2) (layer "F.Cu") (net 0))
 (segment (start 145.465678 98.647658) (end 143.00802 96.19) (width 0.2) (layer "F.Cu") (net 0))
 (segment (start 145.112124 99.001212) (end 141.381212 99.001212) (width 0.2) (layer "F.Cu") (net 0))
 (segment (start 146.172785 97.940551) (end 142.75 94.517766) (width 0.2) (layer "F.Cu") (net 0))
 (segment (start 151.352342 104.534322) (end 153.75 106.93198) (width 0.2) (layer "F.Cu") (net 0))
 (segment (start 146.75 92.860912) (end 146.75 76.43) (width 0.2) (layer "F.Cu") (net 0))
 (segment (start 147.940551 96.172785) (end 147.922785 96.172785) (width 0.2) (layer "F.Cu") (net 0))
 (segment (start 154.75 93.5) (end 154.75 82.55) (width 0.2) (layer "F.Cu") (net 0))
 (segment (start 154.75 106.5) (end 154.75 117.45) (width 0.2) (layer "F.Cu") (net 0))
 (segment (start 145.465678 101.352342) (end 143.00802 103.81) (width 0.2) (layer "F.Cu") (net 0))
 (segment (start 153.473662 102.473662) (end 156.75 105.75) (width 0.2) (layer "F.Cu") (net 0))
 (segment (start 143.75 105.896446) (end 143.75 111.33) (width 0.2) (layer "F.Cu") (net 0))
 (segment (start 153.827215 102.059449) (end 153.827215 102.077215) (width 0.2) (layer "F.Cu") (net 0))
 (segment (start 153.25 123.57) (end 158.89 129.21) (width 0.2) (layer "F.Cu") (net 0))
 (segment (start 144.25 93.896446) (end 144.25 86.63) (width 0.2) (layer "F.Cu") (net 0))
 (segment (start 147.233445 96.879891) (end 144.25 93.896446) (width 0.2) (layer "F.Cu") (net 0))
 (segment (start 147.586998 96.526338) (end 144.75 93.68934) (width 0.2) (layer "F.Cu") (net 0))
 (segment (start 154.25 93.275126) (end 154.25 80.51) (width 0.2) (layer "F.Cu") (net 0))
 (segment (start 142.75 92.75) (end 141.11 91.11) (width 0.2) (layer "F.Cu") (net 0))
 (segment (start 150.998788 104.887876) (end 153.25 107.139088) (width 0.2) (layer "F.Cu") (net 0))
 (segment (start 145.267766 106.5) (end 145.25 106.5) (width 0.2) (layer "F.Cu") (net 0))
 (segment (start 146.526338 97.586998) (end 143.25 94.31066) (width 0.2) (layer "F.Cu") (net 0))
 (segment (start 153.25 76.43) (end 158.89 70.79) (width 0.2) (layer "F.Cu") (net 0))
 (segment (start 153.75 121.53) (end 158.89 126.67) (width 0.2) (layer "F.Cu") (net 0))
 (segment (start 147.586998 103.473662) (end 144.75 106.31066) (width 0.2) (layer "F.Cu") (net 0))
 (segment (start 156.25 88.67) (end 158.89 86.03) (width 0.2) (layer "F.Cu") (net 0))
 (segment (start 147.233445 103.120109) (end 144.25 106.103554) (width 0.2) (layer "F.Cu") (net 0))
 (segment (start 149.001212 95.112124) (end 146.75 92.860912) (width 0.2) (layer "F.Cu") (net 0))
 (segment (start 155.25 115.41) (end 158.89 119.05) (width 0.2) (layer "F.Cu") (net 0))
 (segment (start 148.294105 104.180769) (end 148.294105 104.205895) (width 0.2) (layer "F.Cu") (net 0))
 (segment (start 144.75 106.31066) (end 144.75 115.41) (width 0.2) (layer "F.Cu") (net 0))
 (segment (start 146.25 93.06802) (end 146.25 78.47) (width 0.2) (layer "F.Cu") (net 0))
 (segment (start 154.75 117.45) (end 158.89 121.59) (width 0.2) (layer "F.Cu") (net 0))
 (segment (start 146.75 107.139088) (end 146.75 123.57) (width 0.2) (layer "F.Cu") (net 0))
 (segment (start 141.175126 106.35) (end 141.11 106.35) (width 0.2) (layer "F.Cu") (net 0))
 (segment (start 145.75 93.25) (end 145.75 80.51) (width 0.2) (layer "F.Cu") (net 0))
 (segment (start 156.75 94.25) (end 156.75 90.71) (width 0.2) (layer "F.Cu") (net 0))
 (segment (start 146.25 106.93198) (end 146.25 121.53) (width 0.2) (layer "F.Cu") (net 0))
 (segment (start 156.99198 103.81) (end 158.89 103.81) (width 0.2) (layer "F.Cu") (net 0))
 (segment (start 158.618788 99.001212) (end 158.89 98.73) (width 0.2) (layer "F.Cu") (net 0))
 (segment (start 158.824874 106.35) (end 158.89 106.35) (width 0.2) (layer "F.Cu") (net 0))
 (segment (start 158.618788 100.998788) (end 158.89 101.27) (width 0.2) (layer "F.Cu") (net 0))
 (segment (start 143.75 88.67) (end 141.11 86.03) (width 0.2) (layer "F.Cu") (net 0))
 (segment (start 148.647658 95.465678) (end 146.25 93.06802) (width 0.2) (layer "F.Cu") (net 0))
 (segment (start 154.75 82.55) (end 158.89 78.41) (width 0.2) (layer "F.Cu") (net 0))
 (segment (start 157.25 107.25) (end 158.89 108.89) (width 0.2) (layer "F.Cu") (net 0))
 (segment (start 152.059449 96.172785) (end 152.077215 96.172785) (width 0.2) (layer "F.Cu") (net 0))
 (segment (start 154.25 119.49) (end 158.89 124.13) (width 0.2) (layer "F.Cu") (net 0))
 (segment (start 148.294105 95.794105) (end 145.75 93.25) (width 0.2) (layer "F.Cu") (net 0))
 (segment (start 148.294105 104.205895) (end 145.75 106.75) (width 0.2) (layer "F.Cu") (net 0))
 (segment (start 143.25 109.29) (end 141.11 111.43) (width 0.2) (layer "F.Cu") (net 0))
 (segment (start 145.819231 98.294105) (end 141.175126 93.65) (width 0.2) (layer "F.Cu") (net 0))
 (segment (start 146.526338 102.413002) (end 143.25 105.68934) (width 0.2) (layer "F.Cu") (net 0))
 (segment (start 147.940551 103.827215) (end 145.267766 106.5) (width 0.2) (layer "F.Cu") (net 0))
 (segment (start 156.99198 96.19) (end 158.89 96.19) (width 0.2) (layer "F.Cu") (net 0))
 (segment (start 145.25 82.55) (end 141.11 78.41) (width 0.2) (layer "F.Cu") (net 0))
 (segment (start 155.75 93.896446) (end 155.75 86.63) (width 0.2) (layer "F.Cu") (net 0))
 (segment (start 153.827215 102.077215) (end 157.25 105.5) (width 0.2) (layer "F.Cu") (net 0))
 (segment (start 154.887876 99.001212) (end 158.618788 99.001212) (width 0.2) (layer "F.Cu") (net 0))
 (segment (start 153.473662 97.526338) (end 156.75 94.25) (width 0.2) (layer "F.Cu") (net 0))
 (segment (start 146.172785 102.059449) (end 142.75 105.482234) (width 0.2) (layer "F.Cu") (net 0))
 (segment (start 151.705895 104.180769) (end 154.25 106.724874) (width 0.2) (layer "F.Cu") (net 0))
 (segment (start 157.25 105.5) (end 157.25 107.25) (width 0.2) (layer "F.Cu") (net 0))
 (segment (start 143.75 111.33) (end 141.11 113.97) (width 0.2) (layer "F.Cu") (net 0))
 (segment (start 144.75 84.59) (end 141.11 80.95) (width 0.2) (layer "F.Cu") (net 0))
 (segment (start 153.75 93.06802) (end 153.75 78.47) (width 0.2) (layer "F.Cu") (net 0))
 (segment (start 148.294105 95.819231) (end 148.294105 95.794105) (width 0.2) (layer "F.Cu") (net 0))
 (segment (start 155.75 86.63) (end 158.89 83.49) (width 0.2) (layer "F.Cu") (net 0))
 (segment (start 143.25 90.71) (end 141.11 88.57) (width 0.2) (layer "F.Cu") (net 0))
 (segment (start 146.879891 102.766555) (end 143.75 105.896446) (width 0.2) (layer "F.Cu") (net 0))
 (segment (start 157.25 94.5) (end 157.25 92.75) (width 0.2) (layer "F.Cu") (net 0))
 (segment (start 154.534322 101.352342) (end 156.99198 103.81) (width 0.2) (layer "F.Cu") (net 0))
 (segment (start 153.75 78.47) (end 158.89 73.33) (width 0.2) (layer "F.Cu") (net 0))
 (segment (start 152.059449 103.827215) (end 154.732234 106.5) (width 0.2) (layer "F.Cu") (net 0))
 (segment (start 151.352342 95.465678) (end 153.75 93.06802) (width 0.2) (layer "F.Cu") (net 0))
 (segment (start 144.75 115.41) (end 141.11 119.05) (width 0.2) (layer "F.Cu") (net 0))
 (segment (start 143.75 94.103554) (end 143.75 88.67) (width 0.2) (layer "F.Cu") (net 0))
 (segment (start 155.25 106.31066) (end 155.25 115.41) (width 0.2) (layer "F.Cu") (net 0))
 (segment (start 144.25 106.103554) (end 144.25 113.37) (width 0.2) (layer "F.Cu") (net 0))
 (segment (start 152.077215 96.172785) (end 154.75 93.5) (width 0.2) (layer "F.Cu") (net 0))
 (segment (start 154.180769 101.705895) (end 158.824874 106.35) (width 0.2) (layer "F.Cu") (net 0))
 (segment (start 153.75 106.93198) (end 153.75 121.53) (width 0.2) (layer "F.Cu") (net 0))
 (segment (start 158.824874 93.65) (end 158.89 93.65) (width 0.2) (layer "F.Cu") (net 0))
 (segment (start 155.75 106.103554) (end 155.75 113.37) (width 0.2) (layer "F.Cu") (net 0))
 (segment (start 153.473662 102.413002) (end 153.473662 102.473662) (width 0.2) (layer "F.Cu") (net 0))
 (segment (start 156.75 105.75) (end 156.75 109.29) (width 0.2) (layer "F.Cu") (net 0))
 (segment (start 143.25 105.68934) (end 143.25 109.29) (width 0.2) (layer "F.Cu") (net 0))
 (segment (start 154.25 80.51) (end 158.89 75.87) (width 0.2) (layer "F.Cu") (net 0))
 (segment (start 153.120109 97.233445) (end 156.25 94.103554) (width 0.2) (layer "F.Cu") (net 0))
 (segment (start 144.25 86.63) (end 141.11 83.49) (width 0.2) (layer "F.Cu") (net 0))
 (segment (start 141.175126 93.65) (end 141.11 93.65) (width 0.2) (layer "F.Cu") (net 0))
 (segment (start 145.25 93.5) (end 145.25 82.55) (width 0.2) (layer "F.Cu") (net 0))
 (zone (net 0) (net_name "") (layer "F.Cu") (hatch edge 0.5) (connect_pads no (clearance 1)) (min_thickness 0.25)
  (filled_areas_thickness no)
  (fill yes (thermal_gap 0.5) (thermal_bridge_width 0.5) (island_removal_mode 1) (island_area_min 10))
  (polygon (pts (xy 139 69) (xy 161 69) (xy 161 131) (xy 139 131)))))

